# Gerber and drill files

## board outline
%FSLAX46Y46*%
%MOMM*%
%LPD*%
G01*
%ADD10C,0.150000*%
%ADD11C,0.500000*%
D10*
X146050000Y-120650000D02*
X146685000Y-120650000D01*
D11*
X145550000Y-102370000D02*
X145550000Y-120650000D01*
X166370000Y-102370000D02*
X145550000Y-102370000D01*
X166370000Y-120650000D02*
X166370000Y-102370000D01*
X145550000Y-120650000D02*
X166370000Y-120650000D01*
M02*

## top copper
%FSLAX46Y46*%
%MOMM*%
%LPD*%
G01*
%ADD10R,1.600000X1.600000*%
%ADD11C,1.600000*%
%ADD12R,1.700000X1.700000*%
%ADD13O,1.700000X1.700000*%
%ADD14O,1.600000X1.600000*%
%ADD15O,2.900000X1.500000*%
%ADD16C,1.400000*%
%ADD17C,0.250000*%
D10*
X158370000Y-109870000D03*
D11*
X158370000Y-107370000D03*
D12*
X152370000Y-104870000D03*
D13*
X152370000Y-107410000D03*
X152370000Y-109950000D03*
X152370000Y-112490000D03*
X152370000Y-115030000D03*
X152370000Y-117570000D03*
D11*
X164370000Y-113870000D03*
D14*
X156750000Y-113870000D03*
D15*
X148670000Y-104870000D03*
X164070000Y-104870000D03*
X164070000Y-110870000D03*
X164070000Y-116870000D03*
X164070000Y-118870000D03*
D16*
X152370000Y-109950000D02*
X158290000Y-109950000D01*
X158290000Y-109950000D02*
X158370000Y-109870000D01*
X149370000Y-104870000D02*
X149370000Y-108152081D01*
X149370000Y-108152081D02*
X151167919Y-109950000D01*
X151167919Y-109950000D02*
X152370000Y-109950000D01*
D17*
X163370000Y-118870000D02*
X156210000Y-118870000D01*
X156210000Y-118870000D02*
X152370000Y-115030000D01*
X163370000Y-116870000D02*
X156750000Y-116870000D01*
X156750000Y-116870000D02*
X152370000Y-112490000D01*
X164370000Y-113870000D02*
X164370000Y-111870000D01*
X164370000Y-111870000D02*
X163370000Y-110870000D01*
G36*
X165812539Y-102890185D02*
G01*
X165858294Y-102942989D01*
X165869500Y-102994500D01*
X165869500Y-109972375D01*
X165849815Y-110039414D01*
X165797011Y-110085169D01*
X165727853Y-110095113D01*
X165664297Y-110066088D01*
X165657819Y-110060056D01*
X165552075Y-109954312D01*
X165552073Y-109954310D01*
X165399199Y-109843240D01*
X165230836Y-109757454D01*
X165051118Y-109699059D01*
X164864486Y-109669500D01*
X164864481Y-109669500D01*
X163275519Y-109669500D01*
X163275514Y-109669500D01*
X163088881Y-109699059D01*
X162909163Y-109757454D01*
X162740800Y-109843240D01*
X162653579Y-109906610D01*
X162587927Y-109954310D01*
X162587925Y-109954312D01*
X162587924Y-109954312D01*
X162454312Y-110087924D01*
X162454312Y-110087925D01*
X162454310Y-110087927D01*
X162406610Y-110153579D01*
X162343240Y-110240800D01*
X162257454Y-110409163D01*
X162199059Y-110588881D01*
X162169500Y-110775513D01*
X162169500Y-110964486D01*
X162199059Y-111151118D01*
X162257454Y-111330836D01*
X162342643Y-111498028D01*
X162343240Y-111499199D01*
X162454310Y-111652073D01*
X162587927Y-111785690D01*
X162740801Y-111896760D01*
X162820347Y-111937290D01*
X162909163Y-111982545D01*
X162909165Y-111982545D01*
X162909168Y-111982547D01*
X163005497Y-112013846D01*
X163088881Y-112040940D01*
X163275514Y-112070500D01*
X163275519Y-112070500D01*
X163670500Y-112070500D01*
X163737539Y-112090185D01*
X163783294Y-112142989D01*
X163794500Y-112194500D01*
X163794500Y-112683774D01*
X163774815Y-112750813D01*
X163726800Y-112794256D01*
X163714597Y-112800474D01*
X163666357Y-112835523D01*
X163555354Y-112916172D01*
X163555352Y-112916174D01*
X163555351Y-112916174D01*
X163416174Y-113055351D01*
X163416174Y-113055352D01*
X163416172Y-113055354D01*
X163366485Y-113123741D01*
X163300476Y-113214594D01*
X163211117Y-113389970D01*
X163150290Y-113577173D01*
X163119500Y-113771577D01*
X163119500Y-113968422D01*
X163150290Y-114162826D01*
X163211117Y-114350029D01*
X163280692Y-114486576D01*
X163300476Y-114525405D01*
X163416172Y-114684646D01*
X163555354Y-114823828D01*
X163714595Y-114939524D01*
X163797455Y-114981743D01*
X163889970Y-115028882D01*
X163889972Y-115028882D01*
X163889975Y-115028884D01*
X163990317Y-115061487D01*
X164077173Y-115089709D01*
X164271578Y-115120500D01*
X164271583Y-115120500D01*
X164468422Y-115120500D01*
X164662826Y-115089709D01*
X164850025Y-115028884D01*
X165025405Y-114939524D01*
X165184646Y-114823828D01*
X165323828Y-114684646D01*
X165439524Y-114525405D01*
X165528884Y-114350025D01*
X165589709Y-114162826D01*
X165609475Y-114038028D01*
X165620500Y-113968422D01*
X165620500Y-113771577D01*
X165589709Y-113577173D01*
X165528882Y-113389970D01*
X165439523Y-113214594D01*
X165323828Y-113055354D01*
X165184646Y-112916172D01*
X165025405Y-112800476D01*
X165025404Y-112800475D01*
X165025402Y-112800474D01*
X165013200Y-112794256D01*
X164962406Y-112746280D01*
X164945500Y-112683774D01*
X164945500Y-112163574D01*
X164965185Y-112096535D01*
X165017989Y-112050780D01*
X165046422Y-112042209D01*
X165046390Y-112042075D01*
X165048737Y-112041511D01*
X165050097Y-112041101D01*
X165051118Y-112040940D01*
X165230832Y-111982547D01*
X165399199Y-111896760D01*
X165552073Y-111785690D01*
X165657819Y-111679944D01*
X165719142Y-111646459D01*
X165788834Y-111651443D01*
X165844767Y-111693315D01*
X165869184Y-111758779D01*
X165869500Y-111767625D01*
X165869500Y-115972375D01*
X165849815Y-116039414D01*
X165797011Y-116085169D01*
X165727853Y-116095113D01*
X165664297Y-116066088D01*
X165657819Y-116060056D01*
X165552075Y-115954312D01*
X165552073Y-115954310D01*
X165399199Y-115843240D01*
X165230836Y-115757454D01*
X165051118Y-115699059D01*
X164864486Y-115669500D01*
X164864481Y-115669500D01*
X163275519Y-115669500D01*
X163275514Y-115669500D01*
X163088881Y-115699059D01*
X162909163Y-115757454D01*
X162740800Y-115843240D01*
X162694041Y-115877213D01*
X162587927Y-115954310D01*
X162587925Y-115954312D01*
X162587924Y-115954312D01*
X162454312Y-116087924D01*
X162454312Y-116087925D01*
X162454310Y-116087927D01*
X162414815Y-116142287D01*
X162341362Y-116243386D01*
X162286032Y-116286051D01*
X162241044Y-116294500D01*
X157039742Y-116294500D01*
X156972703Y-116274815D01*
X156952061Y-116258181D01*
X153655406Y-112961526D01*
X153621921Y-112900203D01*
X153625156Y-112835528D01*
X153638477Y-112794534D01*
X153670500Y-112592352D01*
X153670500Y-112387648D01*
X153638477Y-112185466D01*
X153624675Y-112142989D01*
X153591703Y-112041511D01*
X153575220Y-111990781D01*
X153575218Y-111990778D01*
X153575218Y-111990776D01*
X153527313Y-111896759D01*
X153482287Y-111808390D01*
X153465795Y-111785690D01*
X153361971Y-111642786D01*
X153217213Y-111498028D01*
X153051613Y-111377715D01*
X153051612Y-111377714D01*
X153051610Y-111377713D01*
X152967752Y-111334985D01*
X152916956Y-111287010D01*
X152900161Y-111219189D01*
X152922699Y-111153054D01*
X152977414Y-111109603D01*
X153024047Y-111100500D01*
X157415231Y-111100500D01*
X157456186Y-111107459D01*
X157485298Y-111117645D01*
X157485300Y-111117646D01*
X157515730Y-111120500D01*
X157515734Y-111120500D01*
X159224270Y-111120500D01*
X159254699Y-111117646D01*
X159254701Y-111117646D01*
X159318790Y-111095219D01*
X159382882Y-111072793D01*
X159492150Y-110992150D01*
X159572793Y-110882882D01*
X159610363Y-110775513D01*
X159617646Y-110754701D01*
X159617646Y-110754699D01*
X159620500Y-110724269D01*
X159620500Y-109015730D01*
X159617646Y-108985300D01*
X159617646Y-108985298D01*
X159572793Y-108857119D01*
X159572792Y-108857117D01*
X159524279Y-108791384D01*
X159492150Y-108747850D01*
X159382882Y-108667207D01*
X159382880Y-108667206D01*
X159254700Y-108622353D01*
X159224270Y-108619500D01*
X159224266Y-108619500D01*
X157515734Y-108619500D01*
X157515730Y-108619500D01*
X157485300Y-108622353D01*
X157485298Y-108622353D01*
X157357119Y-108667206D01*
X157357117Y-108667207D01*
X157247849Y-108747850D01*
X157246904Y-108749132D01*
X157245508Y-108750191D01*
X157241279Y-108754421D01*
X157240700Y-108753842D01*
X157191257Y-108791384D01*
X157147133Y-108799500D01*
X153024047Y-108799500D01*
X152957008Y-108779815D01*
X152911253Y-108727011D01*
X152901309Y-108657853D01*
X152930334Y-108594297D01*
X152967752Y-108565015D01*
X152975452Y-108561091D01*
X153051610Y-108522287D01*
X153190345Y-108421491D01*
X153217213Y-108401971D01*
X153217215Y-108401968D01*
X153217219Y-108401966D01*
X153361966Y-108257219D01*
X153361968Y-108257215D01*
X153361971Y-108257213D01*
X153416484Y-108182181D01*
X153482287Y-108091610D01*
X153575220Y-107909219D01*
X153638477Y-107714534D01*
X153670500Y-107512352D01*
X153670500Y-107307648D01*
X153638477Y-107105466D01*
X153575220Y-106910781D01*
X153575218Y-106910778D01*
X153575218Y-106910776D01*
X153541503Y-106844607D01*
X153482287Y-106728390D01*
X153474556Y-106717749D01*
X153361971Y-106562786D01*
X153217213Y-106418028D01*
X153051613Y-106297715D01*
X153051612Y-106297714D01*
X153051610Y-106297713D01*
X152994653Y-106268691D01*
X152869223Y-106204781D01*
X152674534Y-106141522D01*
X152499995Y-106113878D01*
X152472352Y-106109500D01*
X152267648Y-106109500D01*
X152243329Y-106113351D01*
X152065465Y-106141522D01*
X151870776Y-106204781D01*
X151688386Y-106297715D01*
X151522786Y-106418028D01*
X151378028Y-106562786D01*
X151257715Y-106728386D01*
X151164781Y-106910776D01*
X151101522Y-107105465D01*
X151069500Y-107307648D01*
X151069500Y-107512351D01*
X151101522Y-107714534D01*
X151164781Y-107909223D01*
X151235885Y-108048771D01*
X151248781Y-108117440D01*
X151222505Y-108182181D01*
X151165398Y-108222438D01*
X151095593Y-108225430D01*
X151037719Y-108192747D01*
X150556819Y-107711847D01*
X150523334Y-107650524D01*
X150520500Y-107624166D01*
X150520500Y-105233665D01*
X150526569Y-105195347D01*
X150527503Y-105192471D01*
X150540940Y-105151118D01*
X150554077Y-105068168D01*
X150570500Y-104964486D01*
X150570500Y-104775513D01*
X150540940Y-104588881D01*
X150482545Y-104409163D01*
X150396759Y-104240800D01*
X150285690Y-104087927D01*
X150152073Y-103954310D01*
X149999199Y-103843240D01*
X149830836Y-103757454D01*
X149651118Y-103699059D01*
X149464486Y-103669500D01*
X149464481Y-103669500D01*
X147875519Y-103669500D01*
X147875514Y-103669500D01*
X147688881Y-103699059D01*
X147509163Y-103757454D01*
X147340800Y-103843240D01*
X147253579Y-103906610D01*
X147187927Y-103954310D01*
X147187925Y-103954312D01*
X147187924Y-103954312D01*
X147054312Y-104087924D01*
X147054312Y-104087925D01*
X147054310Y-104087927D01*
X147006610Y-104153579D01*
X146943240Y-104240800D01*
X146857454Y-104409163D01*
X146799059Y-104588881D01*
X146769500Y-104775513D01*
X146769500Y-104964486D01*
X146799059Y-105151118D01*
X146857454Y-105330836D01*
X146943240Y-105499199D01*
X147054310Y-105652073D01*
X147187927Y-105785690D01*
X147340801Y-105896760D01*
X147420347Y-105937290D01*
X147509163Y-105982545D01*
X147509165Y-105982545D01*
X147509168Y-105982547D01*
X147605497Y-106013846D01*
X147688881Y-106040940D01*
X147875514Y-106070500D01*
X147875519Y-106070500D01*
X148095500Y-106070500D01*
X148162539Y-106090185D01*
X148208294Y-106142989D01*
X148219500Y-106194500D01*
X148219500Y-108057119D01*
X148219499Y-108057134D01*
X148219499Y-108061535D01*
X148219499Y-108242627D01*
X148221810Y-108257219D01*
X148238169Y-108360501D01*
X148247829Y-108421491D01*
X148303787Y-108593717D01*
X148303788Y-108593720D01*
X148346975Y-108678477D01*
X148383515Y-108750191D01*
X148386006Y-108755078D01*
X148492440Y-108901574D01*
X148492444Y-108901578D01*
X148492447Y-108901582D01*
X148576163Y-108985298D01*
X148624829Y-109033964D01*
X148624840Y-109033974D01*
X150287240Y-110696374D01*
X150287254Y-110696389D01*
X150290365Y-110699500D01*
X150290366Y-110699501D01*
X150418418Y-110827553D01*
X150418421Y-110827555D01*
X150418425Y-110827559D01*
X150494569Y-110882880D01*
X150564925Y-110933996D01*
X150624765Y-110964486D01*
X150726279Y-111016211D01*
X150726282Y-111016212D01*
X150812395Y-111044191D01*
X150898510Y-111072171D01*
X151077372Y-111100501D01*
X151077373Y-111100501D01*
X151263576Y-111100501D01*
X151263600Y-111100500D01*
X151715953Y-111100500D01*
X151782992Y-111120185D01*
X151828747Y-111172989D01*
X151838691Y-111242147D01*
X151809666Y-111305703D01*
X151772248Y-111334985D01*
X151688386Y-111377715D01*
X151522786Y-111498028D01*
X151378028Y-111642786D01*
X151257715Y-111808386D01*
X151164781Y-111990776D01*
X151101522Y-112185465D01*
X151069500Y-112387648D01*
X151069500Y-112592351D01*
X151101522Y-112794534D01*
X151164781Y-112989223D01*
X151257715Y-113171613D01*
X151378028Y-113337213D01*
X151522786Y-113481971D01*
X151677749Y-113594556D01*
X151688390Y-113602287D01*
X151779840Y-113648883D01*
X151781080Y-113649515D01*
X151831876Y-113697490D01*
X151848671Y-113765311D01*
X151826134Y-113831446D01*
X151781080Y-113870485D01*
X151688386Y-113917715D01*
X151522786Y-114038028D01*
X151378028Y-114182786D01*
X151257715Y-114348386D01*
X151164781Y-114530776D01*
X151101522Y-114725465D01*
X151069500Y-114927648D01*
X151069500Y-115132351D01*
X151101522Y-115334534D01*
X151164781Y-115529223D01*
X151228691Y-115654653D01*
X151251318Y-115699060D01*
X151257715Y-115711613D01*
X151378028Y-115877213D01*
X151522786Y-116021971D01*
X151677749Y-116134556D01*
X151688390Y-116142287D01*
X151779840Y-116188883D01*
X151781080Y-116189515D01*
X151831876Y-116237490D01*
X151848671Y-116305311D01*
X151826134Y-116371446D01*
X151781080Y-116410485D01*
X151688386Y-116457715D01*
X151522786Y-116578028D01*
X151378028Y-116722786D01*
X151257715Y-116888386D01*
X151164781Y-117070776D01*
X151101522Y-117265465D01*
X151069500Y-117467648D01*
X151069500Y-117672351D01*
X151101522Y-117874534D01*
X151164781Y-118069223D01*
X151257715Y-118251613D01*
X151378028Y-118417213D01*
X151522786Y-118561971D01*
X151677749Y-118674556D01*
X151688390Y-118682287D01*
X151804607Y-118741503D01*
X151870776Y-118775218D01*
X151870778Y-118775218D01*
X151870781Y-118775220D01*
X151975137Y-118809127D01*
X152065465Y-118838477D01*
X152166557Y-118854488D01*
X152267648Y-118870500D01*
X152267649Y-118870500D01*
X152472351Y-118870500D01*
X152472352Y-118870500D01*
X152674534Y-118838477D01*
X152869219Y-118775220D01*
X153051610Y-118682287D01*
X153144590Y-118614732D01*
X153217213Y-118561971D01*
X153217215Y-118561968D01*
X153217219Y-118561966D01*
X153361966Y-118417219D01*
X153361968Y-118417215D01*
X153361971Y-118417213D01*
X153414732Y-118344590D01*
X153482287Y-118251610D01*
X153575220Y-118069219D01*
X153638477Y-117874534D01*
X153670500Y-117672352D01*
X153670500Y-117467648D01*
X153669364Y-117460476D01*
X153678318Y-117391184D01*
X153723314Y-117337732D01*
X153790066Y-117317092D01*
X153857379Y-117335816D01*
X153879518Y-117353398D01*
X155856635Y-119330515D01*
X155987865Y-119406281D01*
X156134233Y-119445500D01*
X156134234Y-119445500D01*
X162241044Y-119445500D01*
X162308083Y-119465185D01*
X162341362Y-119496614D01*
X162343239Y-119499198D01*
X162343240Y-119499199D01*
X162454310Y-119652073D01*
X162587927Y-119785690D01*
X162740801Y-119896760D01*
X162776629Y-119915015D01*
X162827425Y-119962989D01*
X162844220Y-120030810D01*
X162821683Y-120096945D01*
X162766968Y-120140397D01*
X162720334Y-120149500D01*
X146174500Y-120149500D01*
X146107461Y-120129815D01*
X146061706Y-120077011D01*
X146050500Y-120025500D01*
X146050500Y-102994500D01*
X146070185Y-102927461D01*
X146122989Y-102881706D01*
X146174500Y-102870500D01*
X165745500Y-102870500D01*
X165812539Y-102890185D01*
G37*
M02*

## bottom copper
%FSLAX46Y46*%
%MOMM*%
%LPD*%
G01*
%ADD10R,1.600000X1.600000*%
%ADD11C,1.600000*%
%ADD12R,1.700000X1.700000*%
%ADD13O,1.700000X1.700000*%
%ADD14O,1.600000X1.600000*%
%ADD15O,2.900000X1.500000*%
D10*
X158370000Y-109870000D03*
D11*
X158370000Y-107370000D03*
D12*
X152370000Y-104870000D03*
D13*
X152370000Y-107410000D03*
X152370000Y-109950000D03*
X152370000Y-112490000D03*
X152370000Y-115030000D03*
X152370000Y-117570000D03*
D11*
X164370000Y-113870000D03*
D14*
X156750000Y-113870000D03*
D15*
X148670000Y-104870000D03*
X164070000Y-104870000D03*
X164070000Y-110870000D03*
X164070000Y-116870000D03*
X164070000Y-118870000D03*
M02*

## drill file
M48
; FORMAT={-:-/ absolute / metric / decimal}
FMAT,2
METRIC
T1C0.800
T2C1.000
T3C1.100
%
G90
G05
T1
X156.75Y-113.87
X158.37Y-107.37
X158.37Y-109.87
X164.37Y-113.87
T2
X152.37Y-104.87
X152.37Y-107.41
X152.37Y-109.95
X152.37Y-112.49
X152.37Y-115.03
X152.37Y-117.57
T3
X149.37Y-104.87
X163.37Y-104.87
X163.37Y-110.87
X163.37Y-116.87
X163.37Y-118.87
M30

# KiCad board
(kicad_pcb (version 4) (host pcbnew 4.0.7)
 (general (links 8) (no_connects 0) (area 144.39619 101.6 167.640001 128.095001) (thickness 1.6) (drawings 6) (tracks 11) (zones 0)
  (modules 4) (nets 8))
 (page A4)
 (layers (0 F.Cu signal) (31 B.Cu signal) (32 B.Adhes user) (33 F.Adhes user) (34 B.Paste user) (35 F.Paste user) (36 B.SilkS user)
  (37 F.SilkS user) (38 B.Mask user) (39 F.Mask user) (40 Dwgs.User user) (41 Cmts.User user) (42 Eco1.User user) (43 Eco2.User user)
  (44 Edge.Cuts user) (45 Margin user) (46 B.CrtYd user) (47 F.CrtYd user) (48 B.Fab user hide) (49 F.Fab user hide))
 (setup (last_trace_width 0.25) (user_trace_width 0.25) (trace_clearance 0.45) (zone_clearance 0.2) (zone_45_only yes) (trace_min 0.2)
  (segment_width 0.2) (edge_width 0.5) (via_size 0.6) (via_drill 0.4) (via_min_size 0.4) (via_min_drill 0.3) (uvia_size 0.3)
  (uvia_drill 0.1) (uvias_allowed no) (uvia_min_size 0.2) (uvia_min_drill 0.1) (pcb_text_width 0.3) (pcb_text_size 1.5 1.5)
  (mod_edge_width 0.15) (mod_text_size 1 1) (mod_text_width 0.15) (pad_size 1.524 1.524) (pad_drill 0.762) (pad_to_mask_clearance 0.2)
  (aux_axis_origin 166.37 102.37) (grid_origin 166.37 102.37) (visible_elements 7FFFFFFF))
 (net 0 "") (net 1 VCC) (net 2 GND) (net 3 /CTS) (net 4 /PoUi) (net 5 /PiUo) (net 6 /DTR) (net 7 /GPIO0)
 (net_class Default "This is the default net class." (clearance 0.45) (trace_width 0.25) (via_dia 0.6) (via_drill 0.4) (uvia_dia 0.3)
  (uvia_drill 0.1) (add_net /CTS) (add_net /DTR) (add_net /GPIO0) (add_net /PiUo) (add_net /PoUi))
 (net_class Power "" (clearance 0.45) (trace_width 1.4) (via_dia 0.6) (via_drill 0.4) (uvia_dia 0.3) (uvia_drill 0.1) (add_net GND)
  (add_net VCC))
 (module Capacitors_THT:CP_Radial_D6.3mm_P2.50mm (layer F.Cu) (at 158.37 109.87 90)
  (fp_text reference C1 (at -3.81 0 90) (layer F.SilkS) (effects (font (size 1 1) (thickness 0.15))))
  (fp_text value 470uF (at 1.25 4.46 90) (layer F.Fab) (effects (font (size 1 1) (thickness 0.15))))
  (pad 1 thru_hole rect (at 0 0 90) (size 1.6 1.6) (drill 0.8) (layers *.Cu *.Mask) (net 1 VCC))
  (pad 2 thru_hole circle (at 2.5 0 90) (size 1.6 1.6) (drill 0.8) (layers *.Cu *.Mask) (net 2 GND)))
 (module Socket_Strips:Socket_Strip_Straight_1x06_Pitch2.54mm (layer F.Cu) (at 152.37 104.87)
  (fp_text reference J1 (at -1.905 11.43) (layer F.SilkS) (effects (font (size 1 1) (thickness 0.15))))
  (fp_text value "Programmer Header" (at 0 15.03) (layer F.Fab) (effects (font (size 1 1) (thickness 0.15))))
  (pad 1 thru_hole rect (at 0 0) (size 1.7 1.7) (drill 1) (layers *.Cu *.Mask) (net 2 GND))
  (pad 2 thru_hole oval (at 0 2.54) (size 1.7 1.7) (drill 1) (layers *.Cu *.Mask) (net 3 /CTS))
  (pad 3 thru_hole oval (at 0 5.08) (size 1.7 1.7) (drill 1) (layers *.Cu *.Mask) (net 1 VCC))
  (pad 4 thru_hole oval (at 0 7.62) (size 1.7 1.7) (drill 1) (layers *.Cu *.Mask) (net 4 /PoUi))
  (pad 5 thru_hole oval (at 0 10.16) (size 1.7 1.7) (drill 1) (layers *.Cu *.Mask) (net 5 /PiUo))
  (pad 6 thru_hole oval (at 0 12.7) (size 1.7 1.7) (drill 1) (layers *.Cu *.Mask) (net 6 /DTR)))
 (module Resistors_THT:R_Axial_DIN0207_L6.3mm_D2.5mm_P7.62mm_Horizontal (layer F.Cu) (at 164.37 113.87 180)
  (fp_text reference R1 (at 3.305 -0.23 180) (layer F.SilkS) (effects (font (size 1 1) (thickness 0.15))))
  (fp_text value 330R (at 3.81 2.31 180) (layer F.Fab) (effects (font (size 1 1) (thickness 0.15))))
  (pad 1 thru_hole circle (at 0 0 180) (size 1.6 1.6) (drill 0.8) (layers *.Cu *.Mask) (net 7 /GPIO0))
  (pad 2 thru_hole oval (at 7.62 0 180) (size 1.6 1.6) (drill 0.8) (layers *.Cu *.Mask) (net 2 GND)))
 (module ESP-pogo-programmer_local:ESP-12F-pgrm (layer B.Cu) (at 149.37 118.87)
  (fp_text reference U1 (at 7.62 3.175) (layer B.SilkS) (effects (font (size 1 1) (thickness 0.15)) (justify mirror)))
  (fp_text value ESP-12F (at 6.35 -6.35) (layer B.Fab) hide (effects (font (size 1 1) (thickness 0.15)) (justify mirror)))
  (pad 8 thru_hole oval (at 0 -14) (size 2.9 1.5) (drill 1.1 (offset -0.7 0)) (layers *.Cu *.Mask B.SilkS) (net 1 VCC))
  (pad 9 thru_hole oval (at 14 -14) (size 2.9 1.5) (drill 1.1 (offset 0.7 0)) (layers *.Cu *.Mask B.SilkS) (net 2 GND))
  (pad 12 thru_hole oval (at 14 -8) (size 2.9 1.5) (drill 1.1 (offset 0.7 0)) (layers *.Cu *.Mask B.SilkS) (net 7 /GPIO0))
  (pad 15 thru_hole oval (at 14 -2) (size 2.9 1.5) (drill 1.1 (offset 0.7 0)) (layers *.Cu *.Mask B.SilkS) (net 4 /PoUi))
  (pad 16 thru_hole oval (at 14 0) (size 2.9 1.5) (drill 1.1 (offset 0.7 0)) (layers *.Cu *.Mask B.SilkS) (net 5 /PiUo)))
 (gr_line (start 146.05 120.65) (end 146.685 120.65) (angle 90) (layer Edge.Cuts) (width 0.15))
 (gr_line (start 145.55 102.37) (end 145.55 120.65) (angle 90) (layer Edge.Cuts) (width 0.5))
 (gr_line (start 166.37 102.37) (end 145.55 102.37) (angle 90) (layer Edge.Cuts) (width 0.5))
 (gr_line (start 166.37 120.65) (end 166.37 102.37) (angle 90) (layer Edge.Cuts) (width 0.5))
 (gr_line (start 145.55 120.65) (end 166.37 120.65) (angle 90) (layer Edge.Cuts) (width 0.5))
 (segment (start 152.37 109.95) (end 158.29 109.95) (width 1.4) (layer F.Cu) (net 1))
 (segment (start 158.29 109.95) (end 158.37 109.87) (width 1.4) (layer F.Cu) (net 1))
 (segment (start 149.37 104.87) (end 149.37 108.152081) (width 1.4) (layer F.Cu) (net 1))
 (segment (start 149.37 108.152081) (end 151.167919 109.95) (width 1.4) (layer F.Cu) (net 1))
 (segment (start 151.167919 109.95) (end 152.37 109.95) (width 1.4) (layer F.Cu) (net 1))
 (segment (start 163.37 118.87) (end 156.21 118.87) (width 0.25) (layer F.Cu) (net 5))
 (segment (start 156.21 118.87) (end 152.37 115.03) (width 0.25) (layer F.Cu) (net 5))
 (segment (start 163.37 116.87) (end 156.75 116.87) (width 0.25) (layer F.Cu) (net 4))
 (segment (start 156.75 116.87) (end 152.37 112.49) (width 0.25) (layer F.Cu) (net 4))
 (segment (start 164.37 113.87) (end 164.37 111.87) (width 0.25) (layer F.Cu) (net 7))
 (segment (start 164.37 111.87) (end 163.37 110.87) (width 0.25) (layer F.Cu) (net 7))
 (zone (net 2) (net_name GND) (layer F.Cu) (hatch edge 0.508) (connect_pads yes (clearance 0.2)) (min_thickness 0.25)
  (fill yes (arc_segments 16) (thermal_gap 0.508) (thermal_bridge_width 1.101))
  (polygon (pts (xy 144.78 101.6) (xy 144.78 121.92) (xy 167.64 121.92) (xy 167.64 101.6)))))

